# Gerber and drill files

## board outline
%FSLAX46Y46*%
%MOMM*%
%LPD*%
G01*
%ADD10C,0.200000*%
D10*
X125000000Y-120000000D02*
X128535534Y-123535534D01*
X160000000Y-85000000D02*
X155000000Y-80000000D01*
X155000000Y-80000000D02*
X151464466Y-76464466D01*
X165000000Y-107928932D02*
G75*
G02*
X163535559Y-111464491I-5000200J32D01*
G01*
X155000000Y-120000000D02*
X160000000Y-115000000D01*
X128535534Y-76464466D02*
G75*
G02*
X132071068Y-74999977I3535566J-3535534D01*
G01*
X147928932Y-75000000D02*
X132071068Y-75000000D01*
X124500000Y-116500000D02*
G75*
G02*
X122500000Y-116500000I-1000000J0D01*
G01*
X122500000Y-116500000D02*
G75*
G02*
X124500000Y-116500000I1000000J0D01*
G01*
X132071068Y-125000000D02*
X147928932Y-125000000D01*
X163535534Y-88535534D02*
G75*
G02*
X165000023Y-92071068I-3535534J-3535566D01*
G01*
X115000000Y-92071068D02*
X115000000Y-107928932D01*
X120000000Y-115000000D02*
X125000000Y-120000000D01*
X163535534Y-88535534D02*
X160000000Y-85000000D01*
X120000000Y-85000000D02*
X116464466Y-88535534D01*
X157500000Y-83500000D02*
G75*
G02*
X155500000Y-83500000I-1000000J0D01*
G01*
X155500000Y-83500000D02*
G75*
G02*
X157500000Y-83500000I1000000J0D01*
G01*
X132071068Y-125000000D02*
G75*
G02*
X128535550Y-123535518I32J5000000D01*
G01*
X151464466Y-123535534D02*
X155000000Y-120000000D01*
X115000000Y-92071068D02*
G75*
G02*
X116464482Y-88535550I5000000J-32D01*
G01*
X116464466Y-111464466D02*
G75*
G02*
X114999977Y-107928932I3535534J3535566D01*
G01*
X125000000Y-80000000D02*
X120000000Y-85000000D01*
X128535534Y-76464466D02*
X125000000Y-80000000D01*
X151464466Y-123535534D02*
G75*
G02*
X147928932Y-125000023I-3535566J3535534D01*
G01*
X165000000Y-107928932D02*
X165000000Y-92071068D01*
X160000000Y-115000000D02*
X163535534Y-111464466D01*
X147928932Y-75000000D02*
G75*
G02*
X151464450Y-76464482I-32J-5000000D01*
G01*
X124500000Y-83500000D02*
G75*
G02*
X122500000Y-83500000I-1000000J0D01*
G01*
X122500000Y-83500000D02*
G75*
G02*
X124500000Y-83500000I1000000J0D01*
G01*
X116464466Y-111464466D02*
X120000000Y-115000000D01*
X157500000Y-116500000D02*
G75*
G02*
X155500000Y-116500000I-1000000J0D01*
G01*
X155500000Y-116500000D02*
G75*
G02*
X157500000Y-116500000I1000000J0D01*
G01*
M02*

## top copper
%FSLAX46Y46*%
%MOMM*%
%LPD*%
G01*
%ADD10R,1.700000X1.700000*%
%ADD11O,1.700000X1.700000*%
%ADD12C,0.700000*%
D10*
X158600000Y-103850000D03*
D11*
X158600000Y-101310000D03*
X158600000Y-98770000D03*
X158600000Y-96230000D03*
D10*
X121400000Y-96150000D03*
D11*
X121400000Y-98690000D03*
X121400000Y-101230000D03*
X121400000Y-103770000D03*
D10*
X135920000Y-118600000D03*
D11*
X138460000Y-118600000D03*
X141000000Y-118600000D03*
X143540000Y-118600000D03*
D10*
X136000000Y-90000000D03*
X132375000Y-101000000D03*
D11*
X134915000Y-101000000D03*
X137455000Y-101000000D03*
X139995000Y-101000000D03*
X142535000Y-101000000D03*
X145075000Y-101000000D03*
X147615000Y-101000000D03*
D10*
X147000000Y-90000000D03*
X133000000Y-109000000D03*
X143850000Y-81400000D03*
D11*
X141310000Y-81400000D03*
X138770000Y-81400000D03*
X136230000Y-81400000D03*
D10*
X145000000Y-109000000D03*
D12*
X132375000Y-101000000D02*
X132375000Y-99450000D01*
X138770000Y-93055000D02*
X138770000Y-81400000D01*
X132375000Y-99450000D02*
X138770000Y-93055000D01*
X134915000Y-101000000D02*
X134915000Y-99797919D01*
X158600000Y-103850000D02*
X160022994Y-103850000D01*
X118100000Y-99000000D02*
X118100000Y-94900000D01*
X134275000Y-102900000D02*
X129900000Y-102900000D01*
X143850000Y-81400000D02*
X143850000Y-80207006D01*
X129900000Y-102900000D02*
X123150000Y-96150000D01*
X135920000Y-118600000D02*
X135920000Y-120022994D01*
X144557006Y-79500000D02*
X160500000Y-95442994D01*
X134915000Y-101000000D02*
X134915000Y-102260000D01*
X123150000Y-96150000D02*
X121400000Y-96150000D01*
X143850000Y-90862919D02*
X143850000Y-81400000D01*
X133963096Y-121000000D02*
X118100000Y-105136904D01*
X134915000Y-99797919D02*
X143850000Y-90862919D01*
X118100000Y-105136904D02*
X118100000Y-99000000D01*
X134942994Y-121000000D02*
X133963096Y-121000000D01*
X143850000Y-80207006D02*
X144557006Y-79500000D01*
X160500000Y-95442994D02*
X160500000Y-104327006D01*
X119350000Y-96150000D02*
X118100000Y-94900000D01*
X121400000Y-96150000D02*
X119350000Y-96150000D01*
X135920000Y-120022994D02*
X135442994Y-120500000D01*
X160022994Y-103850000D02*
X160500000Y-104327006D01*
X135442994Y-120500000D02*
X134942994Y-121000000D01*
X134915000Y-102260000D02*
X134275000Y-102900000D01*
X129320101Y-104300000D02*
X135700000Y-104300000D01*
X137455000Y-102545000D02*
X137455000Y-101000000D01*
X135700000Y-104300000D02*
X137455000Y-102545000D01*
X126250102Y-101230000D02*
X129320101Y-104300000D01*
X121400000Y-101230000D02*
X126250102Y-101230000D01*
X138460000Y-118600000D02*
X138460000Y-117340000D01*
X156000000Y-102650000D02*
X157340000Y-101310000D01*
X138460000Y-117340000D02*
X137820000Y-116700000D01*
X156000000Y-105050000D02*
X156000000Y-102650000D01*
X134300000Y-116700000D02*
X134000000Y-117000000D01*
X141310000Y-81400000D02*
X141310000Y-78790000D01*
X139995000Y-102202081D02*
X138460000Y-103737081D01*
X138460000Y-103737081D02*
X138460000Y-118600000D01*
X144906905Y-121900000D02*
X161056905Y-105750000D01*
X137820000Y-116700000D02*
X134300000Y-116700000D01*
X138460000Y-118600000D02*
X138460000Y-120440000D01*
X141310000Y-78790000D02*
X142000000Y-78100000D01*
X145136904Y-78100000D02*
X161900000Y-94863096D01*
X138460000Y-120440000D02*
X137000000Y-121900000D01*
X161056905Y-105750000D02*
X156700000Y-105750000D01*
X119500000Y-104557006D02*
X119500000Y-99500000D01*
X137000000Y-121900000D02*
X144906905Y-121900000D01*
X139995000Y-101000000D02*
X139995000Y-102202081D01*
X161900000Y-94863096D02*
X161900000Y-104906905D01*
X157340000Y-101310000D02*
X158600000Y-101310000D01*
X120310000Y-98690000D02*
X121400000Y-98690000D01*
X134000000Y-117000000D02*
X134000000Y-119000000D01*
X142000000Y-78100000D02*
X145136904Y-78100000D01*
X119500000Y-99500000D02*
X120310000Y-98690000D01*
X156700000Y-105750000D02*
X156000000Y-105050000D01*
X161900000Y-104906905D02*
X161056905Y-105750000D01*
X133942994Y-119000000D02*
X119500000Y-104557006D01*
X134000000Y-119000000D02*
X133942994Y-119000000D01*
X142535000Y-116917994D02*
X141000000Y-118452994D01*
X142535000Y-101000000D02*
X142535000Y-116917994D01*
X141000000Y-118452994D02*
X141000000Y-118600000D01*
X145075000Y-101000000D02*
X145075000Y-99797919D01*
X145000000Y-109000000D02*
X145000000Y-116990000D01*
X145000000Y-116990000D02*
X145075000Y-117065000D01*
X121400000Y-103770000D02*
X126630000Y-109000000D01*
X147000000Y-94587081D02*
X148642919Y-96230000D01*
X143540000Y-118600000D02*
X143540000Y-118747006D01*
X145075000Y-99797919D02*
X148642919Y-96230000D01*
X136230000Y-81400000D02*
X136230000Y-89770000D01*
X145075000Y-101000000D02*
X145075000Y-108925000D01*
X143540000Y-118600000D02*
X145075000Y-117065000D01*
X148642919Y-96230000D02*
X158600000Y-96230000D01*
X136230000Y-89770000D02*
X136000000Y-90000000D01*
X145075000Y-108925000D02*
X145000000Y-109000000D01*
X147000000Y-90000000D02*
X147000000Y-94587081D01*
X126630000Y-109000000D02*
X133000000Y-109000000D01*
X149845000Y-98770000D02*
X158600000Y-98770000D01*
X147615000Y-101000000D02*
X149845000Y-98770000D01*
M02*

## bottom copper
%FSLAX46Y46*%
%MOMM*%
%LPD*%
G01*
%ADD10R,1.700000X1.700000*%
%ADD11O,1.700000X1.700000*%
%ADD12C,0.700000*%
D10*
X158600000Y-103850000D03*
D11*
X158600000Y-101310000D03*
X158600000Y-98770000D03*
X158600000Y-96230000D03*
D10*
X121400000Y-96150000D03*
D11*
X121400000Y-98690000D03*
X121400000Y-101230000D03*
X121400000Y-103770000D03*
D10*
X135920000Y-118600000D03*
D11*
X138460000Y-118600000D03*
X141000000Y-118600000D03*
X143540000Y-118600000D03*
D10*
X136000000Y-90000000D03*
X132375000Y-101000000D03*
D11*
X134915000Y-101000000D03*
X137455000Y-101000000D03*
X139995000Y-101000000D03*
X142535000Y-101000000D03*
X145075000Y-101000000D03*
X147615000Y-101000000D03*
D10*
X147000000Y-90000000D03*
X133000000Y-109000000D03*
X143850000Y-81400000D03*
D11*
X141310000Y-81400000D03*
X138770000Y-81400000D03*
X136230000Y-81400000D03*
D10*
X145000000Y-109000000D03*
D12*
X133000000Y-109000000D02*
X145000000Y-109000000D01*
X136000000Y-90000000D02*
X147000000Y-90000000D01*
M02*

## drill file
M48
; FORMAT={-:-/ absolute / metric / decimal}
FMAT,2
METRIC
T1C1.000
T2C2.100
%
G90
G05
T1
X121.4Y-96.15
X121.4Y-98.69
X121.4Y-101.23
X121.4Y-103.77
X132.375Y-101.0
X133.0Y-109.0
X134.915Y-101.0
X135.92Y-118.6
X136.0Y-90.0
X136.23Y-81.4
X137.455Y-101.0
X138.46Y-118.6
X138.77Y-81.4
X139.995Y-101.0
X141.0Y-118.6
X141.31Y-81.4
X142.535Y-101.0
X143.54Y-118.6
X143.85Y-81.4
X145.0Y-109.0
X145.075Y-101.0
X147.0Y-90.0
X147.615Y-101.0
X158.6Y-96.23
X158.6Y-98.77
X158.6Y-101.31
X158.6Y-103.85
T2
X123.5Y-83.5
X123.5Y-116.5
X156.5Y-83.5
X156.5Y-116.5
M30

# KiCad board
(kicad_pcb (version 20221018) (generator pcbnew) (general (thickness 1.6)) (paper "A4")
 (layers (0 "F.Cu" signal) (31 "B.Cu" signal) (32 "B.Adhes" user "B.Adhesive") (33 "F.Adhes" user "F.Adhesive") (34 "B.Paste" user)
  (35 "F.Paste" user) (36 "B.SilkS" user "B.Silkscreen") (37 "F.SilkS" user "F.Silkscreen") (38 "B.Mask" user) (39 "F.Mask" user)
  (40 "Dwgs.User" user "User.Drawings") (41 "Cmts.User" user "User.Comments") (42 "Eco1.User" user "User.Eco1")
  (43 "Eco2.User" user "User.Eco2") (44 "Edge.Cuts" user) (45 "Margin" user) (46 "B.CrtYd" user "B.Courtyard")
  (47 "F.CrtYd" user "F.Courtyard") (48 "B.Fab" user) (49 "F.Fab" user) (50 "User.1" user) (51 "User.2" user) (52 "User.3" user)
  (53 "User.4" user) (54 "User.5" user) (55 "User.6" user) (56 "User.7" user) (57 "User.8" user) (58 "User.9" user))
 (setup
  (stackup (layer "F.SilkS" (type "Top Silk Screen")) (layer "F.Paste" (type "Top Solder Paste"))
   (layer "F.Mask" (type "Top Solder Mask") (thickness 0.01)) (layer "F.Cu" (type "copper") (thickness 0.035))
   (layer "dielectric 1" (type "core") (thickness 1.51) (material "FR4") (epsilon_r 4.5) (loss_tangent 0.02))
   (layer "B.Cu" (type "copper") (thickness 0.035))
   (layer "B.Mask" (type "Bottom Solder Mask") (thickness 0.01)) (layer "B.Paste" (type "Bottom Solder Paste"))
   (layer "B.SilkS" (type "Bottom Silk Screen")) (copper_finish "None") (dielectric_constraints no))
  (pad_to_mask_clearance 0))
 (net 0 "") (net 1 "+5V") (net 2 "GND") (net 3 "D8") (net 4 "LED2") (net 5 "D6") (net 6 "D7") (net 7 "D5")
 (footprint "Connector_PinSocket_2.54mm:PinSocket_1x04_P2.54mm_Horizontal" (layer "F.Cu") (at 158.6 103.85 180)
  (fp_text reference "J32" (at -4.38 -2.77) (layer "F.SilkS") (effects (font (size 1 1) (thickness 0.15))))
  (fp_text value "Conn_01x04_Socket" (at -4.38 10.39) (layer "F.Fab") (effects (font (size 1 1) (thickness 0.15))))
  (pad "1" thru_hole rect (at 0 0 180) (size 1.7 1.7) (drill 1) (layers "*.Cu" "*.Mask") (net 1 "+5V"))
  (pad "2" thru_hole oval (at 0 2.54 180) (size 1.7 1.7) (drill 1) (layers "*.Cu" "*.Mask") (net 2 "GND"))
  (pad "3" thru_hole oval (at 0 5.08 180) (size 1.7 1.7) (drill 1) (layers "*.Cu" "*.Mask") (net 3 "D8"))
  (pad "4" thru_hole oval (at 0 7.62 180) (size 1.7 1.7) (drill 1) (layers "*.Cu" "*.Mask") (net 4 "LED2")))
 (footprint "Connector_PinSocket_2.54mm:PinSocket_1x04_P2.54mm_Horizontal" (layer "F.Cu") (at 121.4 96.15)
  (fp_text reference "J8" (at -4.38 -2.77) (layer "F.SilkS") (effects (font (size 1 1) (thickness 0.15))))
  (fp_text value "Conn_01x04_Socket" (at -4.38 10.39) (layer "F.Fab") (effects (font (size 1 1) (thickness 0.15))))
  (pad "1" thru_hole rect (at 0 0) (size 1.7 1.7) (drill 1) (layers "*.Cu" "*.Mask") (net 1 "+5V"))
  (pad "2" thru_hole oval (at 0 2.54) (size 1.7 1.7) (drill 1) (layers "*.Cu" "*.Mask") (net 2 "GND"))
  (pad "3" thru_hole oval (at 0 5.08) (size 1.7 1.7) (drill 1) (layers "*.Cu" "*.Mask") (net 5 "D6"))
  (pad "4" thru_hole oval (at 0 7.62) (size 1.7 1.7) (drill 1) (layers "*.Cu" "*.Mask") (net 4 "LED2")))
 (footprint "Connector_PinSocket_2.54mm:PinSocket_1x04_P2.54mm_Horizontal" (layer "F.Cu") (at 135.92 118.6 90)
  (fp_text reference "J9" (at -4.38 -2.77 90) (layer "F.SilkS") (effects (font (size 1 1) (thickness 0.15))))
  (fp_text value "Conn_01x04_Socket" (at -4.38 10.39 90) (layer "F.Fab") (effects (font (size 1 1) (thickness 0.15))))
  (pad "1" thru_hole rect (at 0 0 90) (size 1.7 1.7) (drill 1) (layers "*.Cu" "*.Mask") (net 1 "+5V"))
  (pad "2" thru_hole oval (at 0 2.54 90) (size 1.7 1.7) (drill 1) (layers "*.Cu" "*.Mask") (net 2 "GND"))
  (pad "3" thru_hole oval (at 0 5.08 90) (size 1.7 1.7) (drill 1) (layers "*.Cu" "*.Mask") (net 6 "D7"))
  (pad "4" thru_hole oval (at 0 7.62 90) (size 1.7 1.7) (drill 1) (layers "*.Cu" "*.Mask") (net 4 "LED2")))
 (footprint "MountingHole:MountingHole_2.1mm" (layer "F.Cu") (at 123.5 83.5)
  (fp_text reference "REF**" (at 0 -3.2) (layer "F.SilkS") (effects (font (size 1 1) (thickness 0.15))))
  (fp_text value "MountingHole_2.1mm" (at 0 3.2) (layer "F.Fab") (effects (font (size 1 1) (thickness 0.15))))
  (pad "" np_thru_hole circle (at 0 0) (size 2.1 2.1) (drill 2.1) (layers "*.Cu" "*.Mask")))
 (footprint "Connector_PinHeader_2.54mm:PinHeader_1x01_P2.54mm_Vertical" (layer "F.Cu") (at 136 90)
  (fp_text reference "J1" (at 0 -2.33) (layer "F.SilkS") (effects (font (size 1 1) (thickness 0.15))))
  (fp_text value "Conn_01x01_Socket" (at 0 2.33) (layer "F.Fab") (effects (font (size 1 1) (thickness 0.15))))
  (pad "1" thru_hole rect (at 0 0) (size 1.7 1.7) (drill 1) (layers "*.Cu" "*.Mask") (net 4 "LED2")))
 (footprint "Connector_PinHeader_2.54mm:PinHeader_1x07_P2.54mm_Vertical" (layer "F.Cu") (at 132.375 101 90)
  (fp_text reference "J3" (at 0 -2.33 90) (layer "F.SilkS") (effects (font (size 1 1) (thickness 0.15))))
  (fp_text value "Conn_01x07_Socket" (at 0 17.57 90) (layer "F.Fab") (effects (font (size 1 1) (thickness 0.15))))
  (pad "1" thru_hole rect (at 0 0 90) (size 1.7 1.7) (drill 1) (layers "*.Cu" "*.Mask") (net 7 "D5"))
  (pad "2" thru_hole oval (at 0 2.54 90) (size 1.7 1.7) (drill 1) (layers "*.Cu" "*.Mask") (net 1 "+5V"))
  (pad "3" thru_hole oval (at 0 5.08 90) (size 1.7 1.7) (drill 1) (layers "*.Cu" "*.Mask") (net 5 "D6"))
  (pad "4" thru_hole oval (at 0 7.62 90) (size 1.7 1.7) (drill 1) (layers "*.Cu" "*.Mask") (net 2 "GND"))
  (pad "5" thru_hole oval (at 0 10.16 90) (size 1.7 1.7) (drill 1) (layers "*.Cu" "*.Mask") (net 6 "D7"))
  (pad "6" thru_hole oval (at 0 12.7 90) (size 1.7 1.7) (drill 1) (layers "*.Cu" "*.Mask") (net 4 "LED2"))
  (pad "7" thru_hole oval (at 0 15.24 90) (size 1.7 1.7) (drill 1) (layers "*.Cu" "*.Mask") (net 3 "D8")))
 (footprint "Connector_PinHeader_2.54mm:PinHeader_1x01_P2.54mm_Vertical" (layer "F.Cu") (at 147 90)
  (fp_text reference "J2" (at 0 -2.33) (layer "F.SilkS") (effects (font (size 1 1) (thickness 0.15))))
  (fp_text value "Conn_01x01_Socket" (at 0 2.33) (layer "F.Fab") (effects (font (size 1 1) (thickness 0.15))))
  (pad "1" thru_hole rect (at 0 0) (size 1.7 1.7) (drill 1) (layers "*.Cu" "*.Mask") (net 4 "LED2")))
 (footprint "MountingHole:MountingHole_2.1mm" (layer "F.Cu") (at 156.5 83.5)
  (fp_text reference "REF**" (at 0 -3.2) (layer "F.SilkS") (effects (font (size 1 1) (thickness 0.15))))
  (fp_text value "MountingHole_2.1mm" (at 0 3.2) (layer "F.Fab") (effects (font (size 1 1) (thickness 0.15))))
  (pad "" np_thru_hole circle (at 0 0) (size 2.1 2.1) (drill 2.1) (layers "F&B.Cu" "*.Mask")))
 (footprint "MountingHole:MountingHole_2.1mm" (layer "F.Cu") (at 123.5 116.5)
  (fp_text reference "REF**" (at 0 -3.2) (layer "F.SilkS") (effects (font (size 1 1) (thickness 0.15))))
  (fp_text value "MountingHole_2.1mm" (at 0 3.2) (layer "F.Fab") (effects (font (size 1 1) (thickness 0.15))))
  (pad "" np_thru_hole circle (at 0 0) (size 2.1 2.1) (drill 2.1) (layers "F&B.Cu" "*.Mask")))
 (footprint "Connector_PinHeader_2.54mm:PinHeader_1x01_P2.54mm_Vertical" (layer "F.Cu") (at 133 109)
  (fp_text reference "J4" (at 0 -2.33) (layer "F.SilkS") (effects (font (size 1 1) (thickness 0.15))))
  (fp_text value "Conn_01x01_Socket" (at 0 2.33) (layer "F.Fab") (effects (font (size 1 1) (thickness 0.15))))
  (pad "1" thru_hole rect (at 0 0) (size 1.7 1.7) (drill 1) (layers "*.Cu" "*.Mask") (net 4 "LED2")))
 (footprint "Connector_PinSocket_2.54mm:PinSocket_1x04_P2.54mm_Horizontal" (layer "F.Cu") (at 143.85 81.4 -90)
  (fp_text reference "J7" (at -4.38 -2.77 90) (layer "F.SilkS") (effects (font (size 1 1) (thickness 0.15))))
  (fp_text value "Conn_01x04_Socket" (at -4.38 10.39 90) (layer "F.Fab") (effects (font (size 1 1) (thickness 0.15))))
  (pad "1" thru_hole rect (at 0 0 270) (size 1.7 1.7) (drill 1) (layers "*.Cu" "*.Mask") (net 1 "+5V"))
  (pad "2" thru_hole oval (at 0 2.54 270) (size 1.7 1.7) (drill 1) (layers "*.Cu" "*.Mask") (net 2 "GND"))
  (pad "3" thru_hole oval (at 0 5.08 270) (size 1.7 1.7) (drill 1) (layers "*.Cu" "*.Mask") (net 7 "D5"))
  (pad "4" thru_hole oval (at 0 7.62 270) (size 1.7 1.7) (drill 1) (layers "*.Cu" "*.Mask") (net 4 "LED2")))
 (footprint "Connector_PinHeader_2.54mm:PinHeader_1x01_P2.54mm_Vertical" (layer "F.Cu") (at 145 109)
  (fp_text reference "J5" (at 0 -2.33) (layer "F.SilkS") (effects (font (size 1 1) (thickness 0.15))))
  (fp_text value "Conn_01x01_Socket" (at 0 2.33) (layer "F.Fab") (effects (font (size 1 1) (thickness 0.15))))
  (pad "1" thru_hole rect (at 0 0) (size 1.7 1.7) (drill 1) (layers "*.Cu" "*.Mask") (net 4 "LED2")))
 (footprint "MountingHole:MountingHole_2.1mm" (layer "F.Cu") (at 156.5 116.5)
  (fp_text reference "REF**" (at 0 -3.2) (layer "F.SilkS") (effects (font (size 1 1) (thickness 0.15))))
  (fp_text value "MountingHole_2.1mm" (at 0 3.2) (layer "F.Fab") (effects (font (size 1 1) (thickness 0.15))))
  (pad "" np_thru_hole circle (at 0 0) (size 2.1 2.1) (drill 2.1) (layers "F&B.Cu" "*.Mask")))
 (gr_line (start 125 120) (end 128.535534 123.535534) (stroke (width 0.2) (type solid)) (layer "Edge.Cuts"))
 (gr_line (start 160 85) (end 155 80) (stroke (width 0.2) (type solid)) (layer "Edge.Cuts"))
 (gr_line (start 155 80) (end 151.464466 76.464466) (stroke (width 0.2) (type solid)) (layer "Edge.Cuts"))
 (gr_arc (start 165 107.928932) (mid 164.619387 109.842342) (end 163.535534 111.464466) (stroke (width 0.2) (type solid))
  (layer "Edge.Cuts"))
 (gr_line (start 155 120) (end 160 115) (stroke (width 0.2) (type solid)) (layer "Edge.Cuts"))
 (gr_arc (start 128.535534 76.464466) (mid 130.157651 75.380602) (end 132.071068 75) (stroke (width 0.2) (type solid)) (layer "Edge.Cuts"))
 (gr_line (start 147.928932 75) (end 132.071068 75) (stroke (width 0.2) (type solid)) (layer "Edge.Cuts"))
 (gr_circle (center 123.5 116.5) (end 124.5 116.5) (stroke (width 0.2) (type solid)) (fill none) (layer "Edge.Cuts"))
 (gr_line (start 132.071068 125) (end 147.928932 125) (stroke (width 0.2) (type solid)) (layer "Edge.Cuts"))
 (gr_arc (start 163.535534 88.535534) (mid 164.619398 90.157651) (end 165 92.071068) (stroke (width 0.2) (type solid)) (layer "Edge.Cuts"))
 (gr_line (start 115 92.071068) (end 115 107.928932) (stroke (width 0.2) (type solid)) (layer "Edge.Cuts"))
 (gr_line (start 120 115) (end 125 120) (stroke (width 0.2) (type solid)) (layer "Edge.Cuts"))
 (gr_line (start 163.535534 88.535534) (end 160 85) (stroke (width 0.2) (type solid)) (layer "Edge.Cuts"))
 (gr_line (start 120 85) (end 116.464466 88.535534) (stroke (width 0.2) (type solid)) (layer "Edge.Cuts"))
 (gr_circle (center 156.5 83.5) (end 157.5 83.5) (stroke (width 0.2) (type solid)) (fill none) (layer "Edge.Cuts"))
 (gr_arc (start 132.071068 125) (mid 130.157651 124.619398) (end 128.535534 123.535534) (stroke (width 0.2) (type solid))
  (layer "Edge.Cuts"))
 (gr_line (start 151.464466 123.535534) (end 155 120) (stroke (width 0.2) (type solid)) (layer "Edge.Cuts"))
 (gr_arc (start 115 92.071068) (mid 115.380602 90.157651) (end 116.464466 88.535534) (stroke (width 0.2) (type solid)) (layer "Edge.Cuts"))
 (gr_arc (start 116.464466 111.464466) (mid 115.380602 109.842349) (end 115 107.928932) (stroke (width 0.2) (type solid))
  (layer "Edge.Cuts"))
 (gr_line (start 125 80) (end 120 85) (stroke (width 0.2) (type solid)) (layer "Edge.Cuts"))
 (gr_line (start 128.535534 76.464466) (end 125 80) (stroke (width 0.2) (type solid)) (layer "Edge.Cuts"))
 (gr_arc (start 151.464466 123.535534) (mid 149.842349 124.619398) (end 147.928932 125) (stroke (width 0.2) (type solid))
  (layer "Edge.Cuts"))
 (gr_line (start 165 107.928932) (end 165 92.071068) (stroke (width 0.2) (type solid)) (layer "Edge.Cuts"))
 (gr_line (start 160 115) (end 163.535534 111.464466) (stroke (width 0.2) (type solid)) (layer "Edge.Cuts"))
 (gr_arc (start 147.928932 75) (mid 149.842349 75.380603) (end 151.464466 76.464466) (stroke (width 0.2) (type solid)) (layer "Edge.Cuts"))
 (gr_circle (center 123.5 83.5) (end 124.5 83.5) (stroke (width 0.2) (type solid)) (fill none) (layer "Edge.Cuts"))
 (gr_line (start 116.464466 111.464466) (end 120 115) (stroke (width 0.2) (type solid)) (layer "Edge.Cuts"))
 (gr_circle (center 156.5 116.5) (end 157.5 116.5) (stroke (width 0.2) (type solid)) (fill none) (layer "Edge.Cuts"))
 (segment (start 132.375 101) (end 132.375 99.45) (width 0.7) (layer "F.Cu") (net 7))
 (segment (start 138.77 93.055) (end 138.77 81.4) (width 0.7) (layer "F.Cu") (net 7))
 (segment (start 132.375 99.45) (end 138.77 93.055) (width 0.7) (layer "F.Cu") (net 7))
 (segment (start 134.915 101) (end 134.915 99.797919) (width 0.7) (layer "F.Cu") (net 1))
 (segment (start 158.6 103.85) (end 160.022994 103.85) (width 0.7) (layer "F.Cu") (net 1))
 (segment (start 118.1 99) (end 118.1 94.9) (width 0.7) (layer "F.Cu") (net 1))
 (segment (start 134.275 102.9) (end 129.9 102.9) (width 0.7) (layer "F.Cu") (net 1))
 (segment (start 143.85 81.4) (end 143.85 80.207006) (width 0.7) (layer "F.Cu") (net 1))
 (segment (start 129.9 102.9) (end 123.15 96.15) (width 0.7) (layer "F.Cu") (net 1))
 (segment (start 135.92 118.6) (end 135.92 120.022994) (width 0.7) (layer "F.Cu") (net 1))
 (segment (start 144.557006 79.5) (end 160.5 95.442994) (width 0.7) (layer "F.Cu") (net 1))
 (segment (start 134.915 101) (end 134.915 102.26) (width 0.7) (layer "F.Cu") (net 1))
 (segment (start 123.15 96.15) (end 121.4 96.15) (width 0.7) (layer "F.Cu") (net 1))
 (segment (start 143.85 90.862919) (end 143.85 81.4) (width 0.7) (layer "F.Cu") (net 1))
 (segment (start 133.963096 121) (end 118.1 105.136904) (width 0.7) (layer "F.Cu") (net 1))
 (segment (start 134.915 99.797919) (end 143.85 90.862919) (width 0.7) (layer "F.Cu") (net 1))
 (segment (start 118.1 105.136904) (end 118.1 99) (width 0.7) (layer "F.Cu") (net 1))
 (segment (start 134.942994 121) (end 133.963096 121) (width 0.7) (layer "F.Cu") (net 1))
 (segment (start 143.85 80.207006) (end 144.557006 79.5) (width 0.7) (layer "F.Cu") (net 1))
 (segment (start 160.5 95.442994) (end 160.5 104.327006) (width 0.7) (layer "F.Cu") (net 1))
 (segment (start 119.35 96.15) (end 118.1 94.9) (width 0.7) (layer "F.Cu") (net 1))
 (segment (start 121.4 96.15) (end 119.35 96.15) (width 0.7) (layer "F.Cu") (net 1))
 (segment (start 135.92 120.022994) (end 135.442994 120.5) (width 0.7) (layer "F.Cu") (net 1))
 (segment (start 160.022994 103.85) (end 160.5 104.327006) (width 0.7) (layer "F.Cu") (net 1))
 (segment (start 135.442994 120.5) (end 134.942994 121) (width 0.7) (layer "F.Cu") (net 1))
 (segment (start 134.915 102.26) (end 134.275 102.9) (width 0.7) (layer "F.Cu") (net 1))
 (segment (start 129.320101 104.3) (end 135.7 104.3) (width 0.7) (layer "F.Cu") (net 5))
 (segment (start 137.455 102.545) (end 137.455 101) (width 0.7) (layer "F.Cu") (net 5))
 (segment (start 135.7 104.3) (end 137.455 102.545) (width 0.7) (layer "F.Cu") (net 5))
 (segment (start 126.250102 101.23) (end 129.320101 104.3) (width 0.7) (layer "F.Cu") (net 5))
 (segment (start 121.4 101.23) (end 126.250102 101.23) (width 0.7) (layer "F.Cu") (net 5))
 (segment (start 138.46 118.6) (end 138.46 117.34) (width 0.7) (layer "F.Cu") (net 2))
 (segment (start 156 102.65) (end 157.34 101.31) (width 0.7) (layer "F.Cu") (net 2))
 (segment (start 138.46 117.34) (end 137.82 116.7) (width 0.7) (layer "F.Cu") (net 2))
 (segment (start 156 105.05) (end 156 102.65) (width 0.7) (layer "F.Cu") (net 2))
 (segment (start 134.3 116.7) (end 134 117) (width 0.7) (layer "F.Cu") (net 2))
 (segment (start 141.31 81.4) (end 141.31 78.79) (width 0.7) (layer "F.Cu") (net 2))
 (segment (start 139.995 102.202081) (end 138.46 103.737081) (width 0.7) (layer "F.Cu") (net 2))
 (segment (start 138.46 103.737081) (end 138.46 118.6) (width 0.7) (layer "F.Cu") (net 2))
 (segment (start 144.906905 121.9) (end 161.056905 105.75) (width 0.7) (layer "F.Cu") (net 2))
 (segment (start 137.82 116.7) (end 134.3 116.7) (width 0.7) (layer "F.Cu") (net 2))
 (segment (start 138.46 118.6) (end 138.46 120.44) (width 0.7) (layer "F.Cu") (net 2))
 (segment (start 141.31 78.79) (end 142 78.1) (width 0.7) (layer "F.Cu") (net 2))
 (segment (start 145.136904 78.1) (end 161.9 94.863096) (width 0.7) (layer "F.Cu") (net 2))
 (segment (start 138.46 120.44) (end 137 121.9) (width 0.7) (layer "F.Cu") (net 2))
 (segment (start 161.056905 105.75) (end 156.7 105.75) (width 0.7) (layer "F.Cu") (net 2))
 (segment (start 119.5 104.557006) (end 119.5 99.5) (width 0.7) (layer "F.Cu") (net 2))
 (segment (start 137 121.9) (end 144.906905 121.9) (width 0.7) (layer "F.Cu") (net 2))
 (segment (start 139.995 101) (end 139.995 102.202081) (width 0.7) (layer "F.Cu") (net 2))
 (segment (start 161.9 94.863096) (end 161.9 104.906905) (width 0.7) (layer "F.Cu") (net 2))
 (segment (start 157.34 101.31) (end 158.6 101.31) (width 0.7) (layer "F.Cu") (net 2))
 (segment (start 120.31 98.69) (end 121.4 98.69) (width 0.7) (layer "F.Cu") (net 2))
 (segment (start 134 117) (end 134 119) (width 0.7) (layer "F.Cu") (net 2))
 (segment (start 142 78.1) (end 145.136904 78.1) (width 0.7) (layer "F.Cu") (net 2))
 (segment (start 119.5 99.5) (end 120.31 98.69) (width 0.7) (layer "F.Cu") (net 2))
 (segment (start 156.7 105.75) (end 156 105.05) (width 0.7) (layer "F.Cu") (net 2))
 (segment (start 161.9 104.906905) (end 161.056905 105.75) (width 0.7) (layer "F.Cu") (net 2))
 (segment (start 133.942994 119) (end 119.5 104.557006) (width 0.7) (layer "F.Cu") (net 2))
 (segment (start 134 119) (end 133.942994 119) (width 0.7) (layer "F.Cu") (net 2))
 (segment (start 142.535 116.917994) (end 141 118.452994) (width 0.7) (layer "F.Cu") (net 6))
 (segment (start 142.535 101) (end 142.535 116.917994) (width 0.7) (layer "F.Cu") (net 6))
 (segment (start 141 118.452994) (end 141 118.6) (width 0.7) (layer "F.Cu") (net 6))
 (segment (start 145.075 101) (end 145.075 99.797919) (width 0.7) (layer "F.Cu") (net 4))
 (segment (start 145 109) (end 145 116.99) (width 0.7) (layer "F.Cu") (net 4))
 (segment (start 145 116.99) (end 145.075 117.065) (width 0.7) (layer "F.Cu") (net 4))
 (segment (start 121.4 103.77) (end 126.63 109) (width 0.7) (layer "F.Cu") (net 4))
 (segment (start 147 94.587081) (end 148.642919 96.23) (width 0.7) (layer "F.Cu") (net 4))
 (segment (start 143.54 118.6) (end 143.54 118.747006) (width 0.7) (layer "F.Cu") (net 4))
 (segment (start 145.075 99.797919) (end 148.642919 96.23) (width 0.7) (layer "F.Cu") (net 4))
 (segment (start 136.23 81.4) (end 136.23 89.77) (width 0.7) (layer "F.Cu") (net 4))
 (segment (start 145.075 101) (end 145.075 108.925) (width 0.7) (layer "F.Cu") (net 4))
 (segment (start 143.54 118.6) (end 145.075 117.065) (width 0.7) (layer "F.Cu") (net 4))
 (segment (start 148.642919 96.23) (end 158.6 96.23) (width 0.7) (layer "F.Cu") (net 4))
 (segment (start 136.23 89.77) (end 136 90) (width 0.7) (layer "F.Cu") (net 4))
 (segment (start 145.075 108.925) (end 145 109) (width 0.7) (layer "F.Cu") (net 4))
 (segment (start 147 90) (end 147 94.587081) (width 0.7) (layer "F.Cu") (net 4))
 (segment (start 126.63 109) (end 133 109) (width 0.7) (layer "F.Cu") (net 4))
 (segment (start 133 109) (end 145 109) (width 0.7) (layer "B.Cu") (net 4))
 (segment (start 136 90) (end 147 90) (width 0.7) (layer "B.Cu") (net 4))
 (segment (start 149.845 98.77) (end 158.6 98.77) (width 0.7) (layer "F.Cu") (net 3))
 (segment (start 147.615 101) (end 149.845 98.77) (width 0.7) (layer "F.Cu") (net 3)))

